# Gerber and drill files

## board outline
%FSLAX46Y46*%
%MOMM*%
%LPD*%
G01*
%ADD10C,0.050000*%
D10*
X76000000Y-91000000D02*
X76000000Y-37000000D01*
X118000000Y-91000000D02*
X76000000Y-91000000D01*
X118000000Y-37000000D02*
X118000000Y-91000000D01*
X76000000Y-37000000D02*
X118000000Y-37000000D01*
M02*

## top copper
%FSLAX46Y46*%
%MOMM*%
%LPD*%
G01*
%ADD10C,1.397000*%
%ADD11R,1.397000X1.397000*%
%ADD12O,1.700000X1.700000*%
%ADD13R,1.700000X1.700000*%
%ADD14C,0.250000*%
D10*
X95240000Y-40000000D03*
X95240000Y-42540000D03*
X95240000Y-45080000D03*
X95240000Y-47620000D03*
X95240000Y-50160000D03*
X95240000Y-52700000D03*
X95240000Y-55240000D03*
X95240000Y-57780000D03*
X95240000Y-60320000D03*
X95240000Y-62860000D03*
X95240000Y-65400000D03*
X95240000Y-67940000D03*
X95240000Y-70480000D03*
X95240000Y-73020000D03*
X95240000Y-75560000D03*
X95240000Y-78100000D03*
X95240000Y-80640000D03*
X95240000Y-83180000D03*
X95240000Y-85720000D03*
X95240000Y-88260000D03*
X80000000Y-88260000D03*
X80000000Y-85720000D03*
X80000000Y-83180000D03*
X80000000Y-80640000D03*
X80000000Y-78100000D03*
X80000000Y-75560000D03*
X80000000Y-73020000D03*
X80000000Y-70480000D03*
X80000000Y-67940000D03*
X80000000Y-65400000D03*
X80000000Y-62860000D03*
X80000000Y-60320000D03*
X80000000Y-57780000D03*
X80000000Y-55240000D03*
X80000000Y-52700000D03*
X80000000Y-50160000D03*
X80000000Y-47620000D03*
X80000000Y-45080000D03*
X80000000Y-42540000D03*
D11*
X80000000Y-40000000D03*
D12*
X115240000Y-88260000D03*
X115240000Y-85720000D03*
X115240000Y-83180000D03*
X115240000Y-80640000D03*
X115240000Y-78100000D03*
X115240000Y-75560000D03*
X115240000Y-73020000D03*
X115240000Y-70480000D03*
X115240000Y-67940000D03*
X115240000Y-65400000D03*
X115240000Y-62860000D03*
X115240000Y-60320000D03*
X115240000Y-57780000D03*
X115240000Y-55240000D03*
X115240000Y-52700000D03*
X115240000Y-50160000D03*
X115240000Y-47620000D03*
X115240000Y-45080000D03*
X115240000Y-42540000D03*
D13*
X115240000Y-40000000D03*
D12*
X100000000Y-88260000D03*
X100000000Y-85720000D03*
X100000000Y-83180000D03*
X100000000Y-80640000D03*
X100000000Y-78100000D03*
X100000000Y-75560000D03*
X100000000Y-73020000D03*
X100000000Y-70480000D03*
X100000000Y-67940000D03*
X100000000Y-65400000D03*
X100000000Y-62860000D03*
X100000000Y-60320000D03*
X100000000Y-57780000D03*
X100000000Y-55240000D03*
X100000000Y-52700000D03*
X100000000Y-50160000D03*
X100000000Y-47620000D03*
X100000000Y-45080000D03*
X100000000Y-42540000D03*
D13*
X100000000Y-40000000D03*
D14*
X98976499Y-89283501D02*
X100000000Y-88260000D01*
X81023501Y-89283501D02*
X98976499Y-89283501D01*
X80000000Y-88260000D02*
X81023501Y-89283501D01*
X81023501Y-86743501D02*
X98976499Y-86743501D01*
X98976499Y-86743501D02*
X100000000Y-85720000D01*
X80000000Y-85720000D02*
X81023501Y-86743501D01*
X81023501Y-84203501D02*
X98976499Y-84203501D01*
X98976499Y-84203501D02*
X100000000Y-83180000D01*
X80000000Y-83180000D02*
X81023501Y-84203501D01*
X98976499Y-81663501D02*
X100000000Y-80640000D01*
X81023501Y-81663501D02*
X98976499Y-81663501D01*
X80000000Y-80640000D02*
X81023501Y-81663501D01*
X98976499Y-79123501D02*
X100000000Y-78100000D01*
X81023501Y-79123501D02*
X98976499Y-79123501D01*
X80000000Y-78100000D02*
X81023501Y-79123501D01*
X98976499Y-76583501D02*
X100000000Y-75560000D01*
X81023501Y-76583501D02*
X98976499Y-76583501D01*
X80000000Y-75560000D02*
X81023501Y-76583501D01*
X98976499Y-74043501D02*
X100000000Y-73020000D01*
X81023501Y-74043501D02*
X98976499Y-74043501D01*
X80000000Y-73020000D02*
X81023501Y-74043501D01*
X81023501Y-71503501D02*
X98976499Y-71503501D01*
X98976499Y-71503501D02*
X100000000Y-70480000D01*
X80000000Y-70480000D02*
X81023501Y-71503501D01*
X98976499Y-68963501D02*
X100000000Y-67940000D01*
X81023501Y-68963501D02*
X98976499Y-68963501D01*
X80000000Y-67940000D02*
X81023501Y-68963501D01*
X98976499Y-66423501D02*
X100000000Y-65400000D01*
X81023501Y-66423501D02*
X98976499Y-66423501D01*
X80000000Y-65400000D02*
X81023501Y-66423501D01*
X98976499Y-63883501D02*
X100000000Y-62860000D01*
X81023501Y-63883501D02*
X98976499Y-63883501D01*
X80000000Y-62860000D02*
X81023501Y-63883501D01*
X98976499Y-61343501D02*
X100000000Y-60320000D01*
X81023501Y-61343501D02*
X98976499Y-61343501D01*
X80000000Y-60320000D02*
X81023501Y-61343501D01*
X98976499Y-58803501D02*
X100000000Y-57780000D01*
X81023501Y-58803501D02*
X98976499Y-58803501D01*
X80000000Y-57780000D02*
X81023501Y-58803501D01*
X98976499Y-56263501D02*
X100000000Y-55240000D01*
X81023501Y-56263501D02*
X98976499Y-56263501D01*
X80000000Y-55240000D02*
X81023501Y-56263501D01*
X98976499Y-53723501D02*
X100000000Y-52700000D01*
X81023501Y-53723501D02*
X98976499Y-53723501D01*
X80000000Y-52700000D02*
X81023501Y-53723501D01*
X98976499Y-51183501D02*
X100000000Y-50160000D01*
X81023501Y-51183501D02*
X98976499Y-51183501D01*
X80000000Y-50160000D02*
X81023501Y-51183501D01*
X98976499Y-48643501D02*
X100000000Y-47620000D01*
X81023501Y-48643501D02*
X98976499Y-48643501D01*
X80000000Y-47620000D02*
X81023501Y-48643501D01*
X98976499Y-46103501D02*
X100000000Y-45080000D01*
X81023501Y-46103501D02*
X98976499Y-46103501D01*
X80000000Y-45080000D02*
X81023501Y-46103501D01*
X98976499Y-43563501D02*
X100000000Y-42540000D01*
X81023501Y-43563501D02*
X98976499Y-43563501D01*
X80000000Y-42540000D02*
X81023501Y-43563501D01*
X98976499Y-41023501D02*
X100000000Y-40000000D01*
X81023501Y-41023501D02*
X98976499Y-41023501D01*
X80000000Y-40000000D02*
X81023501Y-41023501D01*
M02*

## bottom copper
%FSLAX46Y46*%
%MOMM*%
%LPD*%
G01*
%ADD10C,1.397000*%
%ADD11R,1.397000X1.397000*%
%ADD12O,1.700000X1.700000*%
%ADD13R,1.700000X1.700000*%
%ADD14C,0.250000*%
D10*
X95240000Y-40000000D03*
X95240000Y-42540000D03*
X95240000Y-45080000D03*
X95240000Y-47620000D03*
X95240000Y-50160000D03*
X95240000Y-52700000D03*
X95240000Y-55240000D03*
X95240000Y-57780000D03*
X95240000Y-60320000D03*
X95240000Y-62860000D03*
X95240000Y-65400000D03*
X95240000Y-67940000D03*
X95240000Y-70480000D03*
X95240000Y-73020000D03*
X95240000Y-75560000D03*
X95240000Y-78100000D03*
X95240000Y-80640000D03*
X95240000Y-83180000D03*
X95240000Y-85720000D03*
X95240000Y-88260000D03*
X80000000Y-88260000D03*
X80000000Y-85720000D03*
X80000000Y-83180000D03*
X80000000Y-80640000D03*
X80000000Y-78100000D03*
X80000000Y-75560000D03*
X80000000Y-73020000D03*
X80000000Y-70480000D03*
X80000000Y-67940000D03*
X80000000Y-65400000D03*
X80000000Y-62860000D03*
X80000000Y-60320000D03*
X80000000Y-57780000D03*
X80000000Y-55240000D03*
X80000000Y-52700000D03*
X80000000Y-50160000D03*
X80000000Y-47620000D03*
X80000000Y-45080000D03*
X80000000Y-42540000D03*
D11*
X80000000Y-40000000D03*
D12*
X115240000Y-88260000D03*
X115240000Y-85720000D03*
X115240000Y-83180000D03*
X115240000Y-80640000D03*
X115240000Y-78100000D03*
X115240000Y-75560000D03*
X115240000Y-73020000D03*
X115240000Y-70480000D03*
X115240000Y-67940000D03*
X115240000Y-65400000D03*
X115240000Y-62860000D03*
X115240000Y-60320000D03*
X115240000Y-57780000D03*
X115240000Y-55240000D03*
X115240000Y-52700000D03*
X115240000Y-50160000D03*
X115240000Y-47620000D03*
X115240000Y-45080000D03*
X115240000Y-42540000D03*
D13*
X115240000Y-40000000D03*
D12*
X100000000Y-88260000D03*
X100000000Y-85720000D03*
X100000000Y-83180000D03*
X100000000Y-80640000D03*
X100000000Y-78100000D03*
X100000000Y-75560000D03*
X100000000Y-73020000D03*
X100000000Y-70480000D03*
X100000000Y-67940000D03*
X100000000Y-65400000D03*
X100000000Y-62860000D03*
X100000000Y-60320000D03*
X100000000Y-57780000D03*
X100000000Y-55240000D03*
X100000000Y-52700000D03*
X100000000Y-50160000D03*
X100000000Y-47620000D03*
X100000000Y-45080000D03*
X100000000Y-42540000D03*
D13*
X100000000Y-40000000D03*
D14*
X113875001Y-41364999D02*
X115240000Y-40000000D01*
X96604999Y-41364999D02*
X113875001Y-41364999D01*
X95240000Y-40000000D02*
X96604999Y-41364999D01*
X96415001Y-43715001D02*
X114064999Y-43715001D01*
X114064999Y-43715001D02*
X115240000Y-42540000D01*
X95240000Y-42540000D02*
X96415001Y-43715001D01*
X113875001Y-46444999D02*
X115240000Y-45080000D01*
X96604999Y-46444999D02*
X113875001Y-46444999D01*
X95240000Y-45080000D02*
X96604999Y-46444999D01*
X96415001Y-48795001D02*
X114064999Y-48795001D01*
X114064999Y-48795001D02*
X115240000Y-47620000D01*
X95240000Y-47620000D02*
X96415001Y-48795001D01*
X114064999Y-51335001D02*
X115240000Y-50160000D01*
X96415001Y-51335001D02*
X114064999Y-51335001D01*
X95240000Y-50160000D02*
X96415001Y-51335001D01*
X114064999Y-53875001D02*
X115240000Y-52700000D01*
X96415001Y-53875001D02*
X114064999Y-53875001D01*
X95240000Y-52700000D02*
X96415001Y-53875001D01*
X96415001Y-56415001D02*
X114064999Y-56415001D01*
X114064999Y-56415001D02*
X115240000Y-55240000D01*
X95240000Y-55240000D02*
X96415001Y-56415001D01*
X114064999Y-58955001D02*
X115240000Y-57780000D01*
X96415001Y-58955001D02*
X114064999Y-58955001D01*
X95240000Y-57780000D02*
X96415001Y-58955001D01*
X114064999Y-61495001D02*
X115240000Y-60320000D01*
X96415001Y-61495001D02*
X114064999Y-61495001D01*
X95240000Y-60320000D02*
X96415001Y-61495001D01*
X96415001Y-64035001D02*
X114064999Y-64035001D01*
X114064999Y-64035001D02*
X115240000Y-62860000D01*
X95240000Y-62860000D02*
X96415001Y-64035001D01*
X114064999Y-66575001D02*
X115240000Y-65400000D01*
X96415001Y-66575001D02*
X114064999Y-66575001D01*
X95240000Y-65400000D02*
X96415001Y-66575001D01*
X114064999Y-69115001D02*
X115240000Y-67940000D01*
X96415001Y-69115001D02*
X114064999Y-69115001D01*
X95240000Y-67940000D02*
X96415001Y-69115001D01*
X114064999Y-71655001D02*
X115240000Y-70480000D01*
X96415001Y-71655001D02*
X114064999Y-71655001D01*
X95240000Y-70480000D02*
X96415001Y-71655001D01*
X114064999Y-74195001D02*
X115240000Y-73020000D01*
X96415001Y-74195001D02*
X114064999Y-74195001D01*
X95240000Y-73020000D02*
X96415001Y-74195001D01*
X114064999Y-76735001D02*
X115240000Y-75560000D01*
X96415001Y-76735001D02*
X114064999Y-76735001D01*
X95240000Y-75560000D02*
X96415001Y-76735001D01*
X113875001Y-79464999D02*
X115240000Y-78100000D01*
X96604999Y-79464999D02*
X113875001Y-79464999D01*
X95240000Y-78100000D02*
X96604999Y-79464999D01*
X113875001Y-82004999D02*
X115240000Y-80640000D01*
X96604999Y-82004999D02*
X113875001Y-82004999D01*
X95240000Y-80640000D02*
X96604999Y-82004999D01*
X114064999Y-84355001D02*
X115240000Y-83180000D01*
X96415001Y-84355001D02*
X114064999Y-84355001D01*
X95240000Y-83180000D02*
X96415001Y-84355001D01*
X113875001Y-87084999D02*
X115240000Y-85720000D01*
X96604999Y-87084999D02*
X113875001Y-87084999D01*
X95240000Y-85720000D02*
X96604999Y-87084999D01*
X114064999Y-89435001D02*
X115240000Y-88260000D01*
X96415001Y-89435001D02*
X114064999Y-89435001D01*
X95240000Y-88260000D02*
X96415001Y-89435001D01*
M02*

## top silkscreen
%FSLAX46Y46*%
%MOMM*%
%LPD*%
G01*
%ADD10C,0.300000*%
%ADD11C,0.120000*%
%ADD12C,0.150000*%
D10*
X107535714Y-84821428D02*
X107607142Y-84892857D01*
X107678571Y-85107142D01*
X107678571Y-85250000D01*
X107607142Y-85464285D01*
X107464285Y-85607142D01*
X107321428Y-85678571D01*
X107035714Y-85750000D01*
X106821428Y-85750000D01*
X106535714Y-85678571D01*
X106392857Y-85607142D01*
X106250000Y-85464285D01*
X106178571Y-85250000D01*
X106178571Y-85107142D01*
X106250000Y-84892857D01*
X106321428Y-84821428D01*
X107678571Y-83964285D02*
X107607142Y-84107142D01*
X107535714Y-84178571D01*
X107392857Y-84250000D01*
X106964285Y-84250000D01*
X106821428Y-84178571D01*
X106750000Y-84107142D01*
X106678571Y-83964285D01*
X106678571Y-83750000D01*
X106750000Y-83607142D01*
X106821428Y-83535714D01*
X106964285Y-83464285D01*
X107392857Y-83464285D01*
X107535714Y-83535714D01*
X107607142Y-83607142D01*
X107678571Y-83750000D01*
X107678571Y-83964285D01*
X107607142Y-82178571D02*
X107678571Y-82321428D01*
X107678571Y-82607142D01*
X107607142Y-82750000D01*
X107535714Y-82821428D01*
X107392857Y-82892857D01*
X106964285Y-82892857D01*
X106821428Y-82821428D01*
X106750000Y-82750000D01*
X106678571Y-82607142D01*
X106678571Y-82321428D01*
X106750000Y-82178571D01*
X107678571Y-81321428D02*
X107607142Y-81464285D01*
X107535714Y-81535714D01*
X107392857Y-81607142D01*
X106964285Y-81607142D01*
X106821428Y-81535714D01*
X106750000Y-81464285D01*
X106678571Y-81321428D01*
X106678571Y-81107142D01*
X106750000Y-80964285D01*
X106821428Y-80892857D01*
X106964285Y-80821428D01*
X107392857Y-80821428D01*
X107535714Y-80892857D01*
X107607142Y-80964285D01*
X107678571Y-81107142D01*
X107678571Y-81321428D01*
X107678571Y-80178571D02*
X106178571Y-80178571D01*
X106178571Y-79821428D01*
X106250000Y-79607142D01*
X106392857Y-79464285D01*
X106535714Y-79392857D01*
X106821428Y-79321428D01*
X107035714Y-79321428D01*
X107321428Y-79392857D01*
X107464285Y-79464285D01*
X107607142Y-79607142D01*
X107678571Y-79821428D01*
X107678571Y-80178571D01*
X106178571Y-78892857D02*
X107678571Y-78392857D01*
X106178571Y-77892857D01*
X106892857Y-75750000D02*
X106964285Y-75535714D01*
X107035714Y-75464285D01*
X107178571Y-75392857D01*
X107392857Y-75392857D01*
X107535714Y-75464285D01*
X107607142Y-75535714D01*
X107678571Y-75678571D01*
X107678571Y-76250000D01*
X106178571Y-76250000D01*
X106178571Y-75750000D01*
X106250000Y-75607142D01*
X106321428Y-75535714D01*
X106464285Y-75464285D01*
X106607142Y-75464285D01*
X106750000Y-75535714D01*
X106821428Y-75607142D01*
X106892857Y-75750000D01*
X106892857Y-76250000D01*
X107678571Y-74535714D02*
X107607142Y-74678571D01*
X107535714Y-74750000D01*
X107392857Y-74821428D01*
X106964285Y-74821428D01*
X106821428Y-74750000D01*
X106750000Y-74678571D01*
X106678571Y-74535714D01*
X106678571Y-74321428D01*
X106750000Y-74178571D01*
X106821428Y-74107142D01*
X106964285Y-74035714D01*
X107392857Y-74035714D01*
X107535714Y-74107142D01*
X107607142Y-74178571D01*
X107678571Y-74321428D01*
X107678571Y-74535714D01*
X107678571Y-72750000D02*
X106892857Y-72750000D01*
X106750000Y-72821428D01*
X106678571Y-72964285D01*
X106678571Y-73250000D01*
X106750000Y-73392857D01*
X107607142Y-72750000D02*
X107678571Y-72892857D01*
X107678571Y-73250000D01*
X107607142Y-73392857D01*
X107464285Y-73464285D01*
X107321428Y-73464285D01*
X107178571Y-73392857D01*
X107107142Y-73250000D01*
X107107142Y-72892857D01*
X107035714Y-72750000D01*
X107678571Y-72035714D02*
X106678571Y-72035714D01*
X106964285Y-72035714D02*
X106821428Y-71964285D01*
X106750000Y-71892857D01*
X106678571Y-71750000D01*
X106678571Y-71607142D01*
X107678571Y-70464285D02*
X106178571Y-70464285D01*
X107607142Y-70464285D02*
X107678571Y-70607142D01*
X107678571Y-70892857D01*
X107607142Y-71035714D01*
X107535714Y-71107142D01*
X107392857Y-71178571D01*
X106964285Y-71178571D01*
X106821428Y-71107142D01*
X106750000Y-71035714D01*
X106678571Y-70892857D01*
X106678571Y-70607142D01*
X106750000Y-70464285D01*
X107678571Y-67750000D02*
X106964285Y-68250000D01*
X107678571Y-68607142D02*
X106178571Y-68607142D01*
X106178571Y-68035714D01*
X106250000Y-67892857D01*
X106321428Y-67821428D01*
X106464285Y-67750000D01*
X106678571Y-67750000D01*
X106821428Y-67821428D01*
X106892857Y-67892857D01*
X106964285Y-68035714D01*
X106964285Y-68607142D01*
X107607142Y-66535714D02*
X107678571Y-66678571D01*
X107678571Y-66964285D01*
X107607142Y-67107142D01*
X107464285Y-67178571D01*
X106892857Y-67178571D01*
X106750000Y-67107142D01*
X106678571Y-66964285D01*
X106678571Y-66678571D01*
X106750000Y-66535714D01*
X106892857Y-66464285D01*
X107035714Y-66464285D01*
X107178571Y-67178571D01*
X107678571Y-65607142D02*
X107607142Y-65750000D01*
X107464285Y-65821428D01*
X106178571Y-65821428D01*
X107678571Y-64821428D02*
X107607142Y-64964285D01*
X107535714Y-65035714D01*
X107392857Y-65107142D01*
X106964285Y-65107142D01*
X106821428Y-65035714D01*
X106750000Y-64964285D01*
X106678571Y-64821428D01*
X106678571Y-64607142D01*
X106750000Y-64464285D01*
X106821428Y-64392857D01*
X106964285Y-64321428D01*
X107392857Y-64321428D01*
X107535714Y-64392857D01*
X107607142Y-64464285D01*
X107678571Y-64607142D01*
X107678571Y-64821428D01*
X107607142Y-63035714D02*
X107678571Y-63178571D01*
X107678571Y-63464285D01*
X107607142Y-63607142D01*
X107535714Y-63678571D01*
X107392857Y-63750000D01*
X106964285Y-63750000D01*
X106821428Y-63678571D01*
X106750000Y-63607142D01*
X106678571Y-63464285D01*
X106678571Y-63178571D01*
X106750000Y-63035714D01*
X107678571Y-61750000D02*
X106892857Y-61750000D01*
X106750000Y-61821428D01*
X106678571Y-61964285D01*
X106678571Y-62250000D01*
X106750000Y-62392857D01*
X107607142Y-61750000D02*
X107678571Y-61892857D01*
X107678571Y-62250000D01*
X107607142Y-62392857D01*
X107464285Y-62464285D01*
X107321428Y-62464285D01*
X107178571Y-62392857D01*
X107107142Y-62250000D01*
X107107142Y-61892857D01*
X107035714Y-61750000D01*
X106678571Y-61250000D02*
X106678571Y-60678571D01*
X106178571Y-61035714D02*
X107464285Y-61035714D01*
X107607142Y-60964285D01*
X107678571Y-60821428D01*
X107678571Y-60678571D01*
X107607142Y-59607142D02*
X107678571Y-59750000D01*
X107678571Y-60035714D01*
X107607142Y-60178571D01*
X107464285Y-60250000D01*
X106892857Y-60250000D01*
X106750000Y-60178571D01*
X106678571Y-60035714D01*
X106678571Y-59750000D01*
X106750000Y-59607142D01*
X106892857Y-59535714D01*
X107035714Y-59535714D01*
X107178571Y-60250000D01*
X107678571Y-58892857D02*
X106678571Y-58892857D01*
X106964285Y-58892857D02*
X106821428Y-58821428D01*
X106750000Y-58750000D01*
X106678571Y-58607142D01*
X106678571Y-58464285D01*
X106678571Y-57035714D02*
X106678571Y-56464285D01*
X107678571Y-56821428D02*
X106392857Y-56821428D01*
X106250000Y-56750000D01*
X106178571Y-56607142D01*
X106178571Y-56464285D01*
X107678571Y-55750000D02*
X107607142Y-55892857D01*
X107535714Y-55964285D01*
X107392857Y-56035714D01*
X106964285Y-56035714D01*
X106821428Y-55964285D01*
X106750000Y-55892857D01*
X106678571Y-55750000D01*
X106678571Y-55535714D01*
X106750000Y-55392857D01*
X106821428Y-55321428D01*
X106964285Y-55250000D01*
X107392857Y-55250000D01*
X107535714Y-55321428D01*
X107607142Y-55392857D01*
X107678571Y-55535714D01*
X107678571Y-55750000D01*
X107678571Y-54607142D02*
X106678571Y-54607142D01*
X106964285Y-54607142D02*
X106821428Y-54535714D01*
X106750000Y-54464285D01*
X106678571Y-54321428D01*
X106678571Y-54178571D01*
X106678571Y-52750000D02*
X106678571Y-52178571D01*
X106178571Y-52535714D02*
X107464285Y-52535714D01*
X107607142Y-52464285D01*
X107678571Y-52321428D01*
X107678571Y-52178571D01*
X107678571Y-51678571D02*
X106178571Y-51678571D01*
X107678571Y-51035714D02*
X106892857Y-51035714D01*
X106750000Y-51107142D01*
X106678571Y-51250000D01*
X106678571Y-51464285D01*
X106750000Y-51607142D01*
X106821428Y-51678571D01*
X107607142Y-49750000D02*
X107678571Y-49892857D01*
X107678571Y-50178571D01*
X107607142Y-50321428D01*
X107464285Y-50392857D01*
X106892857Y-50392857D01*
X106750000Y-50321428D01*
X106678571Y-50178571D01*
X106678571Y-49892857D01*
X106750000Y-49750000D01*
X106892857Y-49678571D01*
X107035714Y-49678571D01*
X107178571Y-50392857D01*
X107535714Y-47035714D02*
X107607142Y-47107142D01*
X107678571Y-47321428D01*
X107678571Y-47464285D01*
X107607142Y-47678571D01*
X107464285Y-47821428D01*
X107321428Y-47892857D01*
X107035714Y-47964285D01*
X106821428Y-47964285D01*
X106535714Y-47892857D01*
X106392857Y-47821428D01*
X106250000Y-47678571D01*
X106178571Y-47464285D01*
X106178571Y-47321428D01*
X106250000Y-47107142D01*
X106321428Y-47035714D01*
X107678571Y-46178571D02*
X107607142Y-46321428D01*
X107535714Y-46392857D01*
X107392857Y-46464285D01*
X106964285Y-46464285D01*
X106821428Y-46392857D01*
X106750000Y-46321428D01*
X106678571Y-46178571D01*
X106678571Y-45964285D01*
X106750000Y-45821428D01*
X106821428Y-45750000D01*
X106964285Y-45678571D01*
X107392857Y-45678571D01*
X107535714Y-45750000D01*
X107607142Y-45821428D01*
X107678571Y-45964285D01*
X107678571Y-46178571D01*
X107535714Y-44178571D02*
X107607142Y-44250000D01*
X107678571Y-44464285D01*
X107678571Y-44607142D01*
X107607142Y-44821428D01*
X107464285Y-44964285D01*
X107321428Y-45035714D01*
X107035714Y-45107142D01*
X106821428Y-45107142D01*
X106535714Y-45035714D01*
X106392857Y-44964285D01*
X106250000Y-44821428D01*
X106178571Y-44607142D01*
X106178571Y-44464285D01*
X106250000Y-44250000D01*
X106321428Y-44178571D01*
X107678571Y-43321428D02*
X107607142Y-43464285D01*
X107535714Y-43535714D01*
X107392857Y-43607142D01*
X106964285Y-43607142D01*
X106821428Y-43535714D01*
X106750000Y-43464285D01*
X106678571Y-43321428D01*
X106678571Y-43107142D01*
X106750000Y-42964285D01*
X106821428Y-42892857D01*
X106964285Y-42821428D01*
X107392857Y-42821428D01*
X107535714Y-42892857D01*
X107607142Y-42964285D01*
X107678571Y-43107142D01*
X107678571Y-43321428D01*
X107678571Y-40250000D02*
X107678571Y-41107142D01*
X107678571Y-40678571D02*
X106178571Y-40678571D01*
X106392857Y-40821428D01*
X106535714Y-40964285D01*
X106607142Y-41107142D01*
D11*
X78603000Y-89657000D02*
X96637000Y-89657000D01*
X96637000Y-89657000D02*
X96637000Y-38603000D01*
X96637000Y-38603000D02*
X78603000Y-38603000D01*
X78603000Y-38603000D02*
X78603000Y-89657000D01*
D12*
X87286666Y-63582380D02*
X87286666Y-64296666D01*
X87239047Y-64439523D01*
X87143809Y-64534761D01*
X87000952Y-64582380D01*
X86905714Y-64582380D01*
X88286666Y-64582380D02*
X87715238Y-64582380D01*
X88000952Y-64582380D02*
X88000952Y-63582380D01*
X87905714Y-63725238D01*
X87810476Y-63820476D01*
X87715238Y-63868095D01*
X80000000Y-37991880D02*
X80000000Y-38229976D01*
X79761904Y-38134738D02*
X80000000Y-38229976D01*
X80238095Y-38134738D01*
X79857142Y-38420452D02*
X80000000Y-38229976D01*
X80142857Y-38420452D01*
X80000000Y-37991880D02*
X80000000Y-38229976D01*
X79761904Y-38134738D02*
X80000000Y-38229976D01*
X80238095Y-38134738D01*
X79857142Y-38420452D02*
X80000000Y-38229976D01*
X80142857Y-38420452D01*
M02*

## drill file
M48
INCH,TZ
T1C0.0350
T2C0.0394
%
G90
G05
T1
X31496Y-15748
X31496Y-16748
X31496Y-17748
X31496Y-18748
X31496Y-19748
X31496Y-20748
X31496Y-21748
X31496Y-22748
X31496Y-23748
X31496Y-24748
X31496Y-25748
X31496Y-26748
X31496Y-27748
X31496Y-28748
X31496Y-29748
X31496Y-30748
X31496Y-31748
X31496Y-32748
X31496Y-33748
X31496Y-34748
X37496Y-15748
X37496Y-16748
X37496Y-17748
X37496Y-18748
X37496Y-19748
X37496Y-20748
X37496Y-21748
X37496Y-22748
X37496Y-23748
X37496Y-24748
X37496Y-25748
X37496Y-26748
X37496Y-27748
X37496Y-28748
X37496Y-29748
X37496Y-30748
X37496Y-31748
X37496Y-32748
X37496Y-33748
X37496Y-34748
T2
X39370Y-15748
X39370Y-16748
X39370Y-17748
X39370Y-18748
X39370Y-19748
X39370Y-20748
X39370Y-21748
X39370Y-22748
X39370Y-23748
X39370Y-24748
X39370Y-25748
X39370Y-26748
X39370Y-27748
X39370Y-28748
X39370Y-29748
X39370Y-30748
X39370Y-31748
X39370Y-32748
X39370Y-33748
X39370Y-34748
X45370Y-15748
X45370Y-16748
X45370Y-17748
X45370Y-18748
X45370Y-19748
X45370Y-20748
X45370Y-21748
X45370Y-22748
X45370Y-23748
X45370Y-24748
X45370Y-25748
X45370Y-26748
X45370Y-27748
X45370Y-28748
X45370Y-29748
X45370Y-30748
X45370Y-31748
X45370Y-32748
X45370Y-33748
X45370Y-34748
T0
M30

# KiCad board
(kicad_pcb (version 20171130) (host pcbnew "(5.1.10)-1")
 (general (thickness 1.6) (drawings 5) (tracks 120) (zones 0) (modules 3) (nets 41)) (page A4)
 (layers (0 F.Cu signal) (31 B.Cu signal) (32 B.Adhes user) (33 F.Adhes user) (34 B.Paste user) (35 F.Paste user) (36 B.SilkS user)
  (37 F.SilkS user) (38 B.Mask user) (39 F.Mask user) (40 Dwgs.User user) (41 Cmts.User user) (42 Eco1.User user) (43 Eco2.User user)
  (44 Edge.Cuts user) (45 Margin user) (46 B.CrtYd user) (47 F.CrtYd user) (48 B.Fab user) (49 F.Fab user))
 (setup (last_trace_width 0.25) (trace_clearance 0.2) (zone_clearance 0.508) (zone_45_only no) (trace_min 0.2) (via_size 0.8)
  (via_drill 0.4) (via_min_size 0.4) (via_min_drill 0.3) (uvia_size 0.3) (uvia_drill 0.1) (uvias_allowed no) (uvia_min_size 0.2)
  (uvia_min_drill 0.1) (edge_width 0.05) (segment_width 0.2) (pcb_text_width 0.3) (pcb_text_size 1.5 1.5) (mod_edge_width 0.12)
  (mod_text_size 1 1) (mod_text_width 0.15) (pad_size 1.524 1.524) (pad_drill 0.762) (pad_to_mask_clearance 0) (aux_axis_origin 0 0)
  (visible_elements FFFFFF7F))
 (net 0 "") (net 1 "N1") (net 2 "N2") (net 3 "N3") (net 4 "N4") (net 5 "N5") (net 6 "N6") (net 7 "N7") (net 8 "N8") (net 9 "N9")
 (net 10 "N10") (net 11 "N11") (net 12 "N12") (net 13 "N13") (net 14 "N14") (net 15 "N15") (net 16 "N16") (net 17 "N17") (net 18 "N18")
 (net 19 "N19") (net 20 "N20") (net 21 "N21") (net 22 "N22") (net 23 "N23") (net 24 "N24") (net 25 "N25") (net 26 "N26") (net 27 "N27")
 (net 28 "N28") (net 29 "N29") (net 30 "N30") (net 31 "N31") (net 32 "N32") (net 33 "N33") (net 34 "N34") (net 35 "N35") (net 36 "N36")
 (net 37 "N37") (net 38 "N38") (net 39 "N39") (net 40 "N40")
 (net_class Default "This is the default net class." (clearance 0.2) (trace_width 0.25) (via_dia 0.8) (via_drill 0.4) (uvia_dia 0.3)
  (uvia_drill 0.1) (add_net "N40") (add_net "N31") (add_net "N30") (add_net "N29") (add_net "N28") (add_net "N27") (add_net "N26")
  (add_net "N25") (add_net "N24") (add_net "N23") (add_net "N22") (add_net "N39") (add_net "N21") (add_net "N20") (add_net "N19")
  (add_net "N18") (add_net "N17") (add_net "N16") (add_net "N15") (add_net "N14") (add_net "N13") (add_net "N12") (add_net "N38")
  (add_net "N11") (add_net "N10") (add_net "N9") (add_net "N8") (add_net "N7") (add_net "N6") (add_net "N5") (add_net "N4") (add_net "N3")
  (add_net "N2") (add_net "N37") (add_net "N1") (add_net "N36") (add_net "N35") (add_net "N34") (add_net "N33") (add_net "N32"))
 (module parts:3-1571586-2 (layer F.Cu) (at 80 40)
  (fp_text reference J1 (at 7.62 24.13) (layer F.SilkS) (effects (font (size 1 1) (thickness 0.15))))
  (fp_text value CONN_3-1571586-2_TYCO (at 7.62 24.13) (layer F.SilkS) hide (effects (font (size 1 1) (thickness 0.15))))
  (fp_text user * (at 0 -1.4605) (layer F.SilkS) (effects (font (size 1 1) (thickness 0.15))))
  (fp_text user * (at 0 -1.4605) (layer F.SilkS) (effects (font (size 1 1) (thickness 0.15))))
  (fp_line (start -1.397 49.657) (end 16.637 49.657) (layer F.SilkS) (width 0.12))
  (fp_line (start 16.637 49.657) (end 16.637 -1.397) (layer F.SilkS) (width 0.12))
  (fp_line (start 16.637 -1.397) (end -1.397 -1.397) (layer F.SilkS) (width 0.12))
  (fp_line (start -1.397 -1.397) (end -1.397 49.657) (layer F.SilkS) (width 0.12))
  (pad 40 thru_hole circle (at 15.24 0) (size 1.397 1.397) (drill 0.889) (layers *.Cu *.Mask) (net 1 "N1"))
  (pad 39 thru_hole circle (at 15.24 2.54) (size 1.397 1.397) (drill 0.889) (layers *.Cu *.Mask) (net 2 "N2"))
  (pad 38 thru_hole circle (at 15.24 5.08) (size 1.397 1.397) (drill 0.889) (layers *.Cu *.Mask) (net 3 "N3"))
  (pad 37 thru_hole circle (at 15.24 7.62) (size 1.397 1.397) (drill 0.889) (layers *.Cu *.Mask) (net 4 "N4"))
  (pad 36 thru_hole circle (at 15.24 10.16) (size 1.397 1.397) (drill 0.889) (layers *.Cu *.Mask) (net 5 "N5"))
  (pad 35 thru_hole circle (at 15.24 12.7) (size 1.397 1.397) (drill 0.889) (layers *.Cu *.Mask) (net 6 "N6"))
  (pad 34 thru_hole circle (at 15.24 15.24) (size 1.397 1.397) (drill 0.889) (layers *.Cu *.Mask) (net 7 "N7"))
  (pad 33 thru_hole circle (at 15.24 17.78) (size 1.397 1.397) (drill 0.889) (layers *.Cu *.Mask) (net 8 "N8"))
  (pad 32 thru_hole circle (at 15.24 20.32) (size 1.397 1.397) (drill 0.889) (layers *.Cu *.Mask) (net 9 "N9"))
  (pad 31 thru_hole circle (at 15.24 22.86) (size 1.397 1.397) (drill 0.889) (layers *.Cu *.Mask) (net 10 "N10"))
  (pad 30 thru_hole circle (at 15.24 25.4) (size 1.397 1.397) (drill 0.889) (layers *.Cu *.Mask) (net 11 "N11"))
  (pad 29 thru_hole circle (at 15.24 27.94) (size 1.397 1.397) (drill 0.889) (layers *.Cu *.Mask) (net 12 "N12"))
  (pad 28 thru_hole circle (at 15.24 30.48) (size 1.397 1.397) (drill 0.889) (layers *.Cu *.Mask) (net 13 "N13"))
  (pad 27 thru_hole circle (at 15.24 33.02) (size 1.397 1.397) (drill 0.889) (layers *.Cu *.Mask) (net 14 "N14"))
  (pad 26 thru_hole circle (at 15.24 35.56) (size 1.397 1.397) (drill 0.889) (layers *.Cu *.Mask) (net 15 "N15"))
  (pad 25 thru_hole circle (at 15.24 38.1) (size 1.397 1.397) (drill 0.889) (layers *.Cu *.Mask) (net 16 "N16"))
  (pad 24 thru_hole circle (at 15.24 40.64) (size 1.397 1.397) (drill 0.889) (layers *.Cu *.Mask) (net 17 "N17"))
  (pad 23 thru_hole circle (at 15.24 43.18) (size 1.397 1.397) (drill 0.889) (layers *.Cu *.Mask) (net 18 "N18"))
  (pad 22 thru_hole circle (at 15.24 45.72) (size 1.397 1.397) (drill 0.889) (layers *.Cu *.Mask) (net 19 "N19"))
  (pad 21 thru_hole circle (at 15.24 48.26) (size 1.397 1.397) (drill 0.889) (layers *.Cu *.Mask) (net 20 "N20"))
  (pad 20 thru_hole circle (at 0 48.26) (size 1.397 1.397) (drill 0.889) (layers *.Cu *.Mask) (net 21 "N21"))
  (pad 19 thru_hole circle (at 0 45.72) (size 1.397 1.397) (drill 0.889) (layers *.Cu *.Mask) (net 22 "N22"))
  (pad 18 thru_hole circle (at 0 43.18) (size 1.397 1.397) (drill 0.889) (layers *.Cu *.Mask) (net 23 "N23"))
  (pad 17 thru_hole circle (at 0 40.64) (size 1.397 1.397) (drill 0.889) (layers *.Cu *.Mask) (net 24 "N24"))
  (pad 16 thru_hole circle (at 0 38.1) (size 1.397 1.397) (drill 0.889) (layers *.Cu *.Mask) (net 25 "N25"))
  (pad 15 thru_hole circle (at 0 35.56) (size 1.397 1.397) (drill 0.889) (layers *.Cu *.Mask) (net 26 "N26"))
  (pad 14 thru_hole circle (at 0 33.02) (size 1.397 1.397) (drill 0.889) (layers *.Cu *.Mask) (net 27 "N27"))
  (pad 13 thru_hole circle (at 0 30.48) (size 1.397 1.397) (drill 0.889) (layers *.Cu *.Mask) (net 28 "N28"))
  (pad 12 thru_hole circle (at 0 27.94) (size 1.397 1.397) (drill 0.889) (layers *.Cu *.Mask) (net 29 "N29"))
  (pad 11 thru_hole circle (at 0 25.4) (size 1.397 1.397) (drill 0.889) (layers *.Cu *.Mask) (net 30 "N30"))
  (pad 10 thru_hole circle (at 0 22.86) (size 1.397 1.397) (drill 0.889) (layers *.Cu *.Mask) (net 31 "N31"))
  (pad 9 thru_hole circle (at 0 20.32) (size 1.397 1.397) (drill 0.889) (layers *.Cu *.Mask) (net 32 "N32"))
  (pad 8 thru_hole circle (at 0 17.78) (size 1.397 1.397) (drill 0.889) (layers *.Cu *.Mask) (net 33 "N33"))
  (pad 7 thru_hole circle (at 0 15.24) (size 1.397 1.397) (drill 0.889) (layers *.Cu *.Mask) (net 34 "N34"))
  (pad 6 thru_hole circle (at 0 12.7) (size 1.397 1.397) (drill 0.889) (layers *.Cu *.Mask) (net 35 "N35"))
  (pad 5 thru_hole circle (at 0 10.16) (size 1.397 1.397) (drill 0.889) (layers *.Cu *.Mask) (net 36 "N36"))
  (pad 4 thru_hole circle (at 0 7.62) (size 1.397 1.397) (drill 0.889) (layers *.Cu *.Mask) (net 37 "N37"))
  (pad 3 thru_hole circle (at 0 5.08) (size 1.397 1.397) (drill 0.889) (layers *.Cu *.Mask) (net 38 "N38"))
  (pad 2 thru_hole circle (at 0 2.54) (size 1.397 1.397) (drill 0.889) (layers *.Cu *.Mask) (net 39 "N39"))
  (pad 1 thru_hole rect (at 0 0) (size 1.397 1.397) (drill 0.889) (layers *.Cu *.Mask) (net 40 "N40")))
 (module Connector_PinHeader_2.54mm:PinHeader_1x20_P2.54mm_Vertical (layer B.Cu) (at 115.24 40 180)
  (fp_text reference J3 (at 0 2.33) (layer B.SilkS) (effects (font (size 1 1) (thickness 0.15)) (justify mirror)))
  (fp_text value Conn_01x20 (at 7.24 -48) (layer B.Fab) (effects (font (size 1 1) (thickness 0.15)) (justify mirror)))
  (pad 20 thru_hole oval (at 0 -48.26 180) (size 1.7 1.7) (drill 1) (layers *.Cu *.Mask) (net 20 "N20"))
  (pad 19 thru_hole oval (at 0 -45.72 180) (size 1.7 1.7) (drill 1) (layers *.Cu *.Mask) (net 19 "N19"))
  (pad 18 thru_hole oval (at 0 -43.18 180) (size 1.7 1.7) (drill 1) (layers *.Cu *.Mask) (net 18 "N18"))
  (pad 17 thru_hole oval (at 0 -40.64 180) (size 1.7 1.7) (drill 1) (layers *.Cu *.Mask) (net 17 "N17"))
  (pad 16 thru_hole oval (at 0 -38.1 180) (size 1.7 1.7) (drill 1) (layers *.Cu *.Mask) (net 16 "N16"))
  (pad 15 thru_hole oval (at 0 -35.56 180) (size 1.7 1.7) (drill 1) (layers *.Cu *.Mask) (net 15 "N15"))
  (pad 14 thru_hole oval (at 0 -33.02 180) (size 1.7 1.7) (drill 1) (layers *.Cu *.Mask) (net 14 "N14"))
  (pad 13 thru_hole oval (at 0 -30.48 180) (size 1.7 1.7) (drill 1) (layers *.Cu *.Mask) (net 13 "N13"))
  (pad 12 thru_hole oval (at 0 -27.94 180) (size 1.7 1.7) (drill 1) (layers *.Cu *.Mask) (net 12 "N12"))
  (pad 11 thru_hole oval (at 0 -25.4 180) (size 1.7 1.7) (drill 1) (layers *.Cu *.Mask) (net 11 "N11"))
  (pad 10 thru_hole oval (at 0 -22.86 180) (size 1.7 1.7) (drill 1) (layers *.Cu *.Mask) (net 10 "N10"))
  (pad 9 thru_hole oval (at 0 -20.32 180) (size 1.7 1.7) (drill 1) (layers *.Cu *.Mask) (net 9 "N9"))
  (pad 8 thru_hole oval (at 0 -17.78 180) (size 1.7 1.7) (drill 1) (layers *.Cu *.Mask) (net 8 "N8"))
  (pad 7 thru_hole oval (at 0 -15.24 180) (size 1.7 1.7) (drill 1) (layers *.Cu *.Mask) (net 7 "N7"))
  (pad 6 thru_hole oval (at 0 -12.7 180) (size 1.7 1.7) (drill 1) (layers *.Cu *.Mask) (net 6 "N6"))
  (pad 5 thru_hole oval (at 0 -10.16 180) (size 1.7 1.7) (drill 1) (layers *.Cu *.Mask) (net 5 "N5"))
  (pad 4 thru_hole oval (at 0 -7.62 180) (size 1.7 1.7) (drill 1) (layers *.Cu *.Mask) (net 4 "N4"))
  (pad 3 thru_hole oval (at 0 -5.08 180) (size 1.7 1.7) (drill 1) (layers *.Cu *.Mask) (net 3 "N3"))
  (pad 2 thru_hole oval (at 0 -2.54 180) (size 1.7 1.7) (drill 1) (layers *.Cu *.Mask) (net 2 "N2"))
  (pad 1 thru_hole rect (at 0 0 180) (size 1.7 1.7) (drill 1) (layers *.Cu *.Mask) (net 1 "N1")))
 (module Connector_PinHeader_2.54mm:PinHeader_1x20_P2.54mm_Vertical (layer B.Cu) (at 100 40 180)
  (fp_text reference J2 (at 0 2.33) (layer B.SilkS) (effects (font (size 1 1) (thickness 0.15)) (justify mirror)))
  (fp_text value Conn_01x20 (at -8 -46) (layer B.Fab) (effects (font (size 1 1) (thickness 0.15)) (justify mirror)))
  (pad 20 thru_hole oval (at 0 -48.26 180) (size 1.7 1.7) (drill 1) (layers *.Cu *.Mask) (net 21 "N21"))
  (pad 19 thru_hole oval (at 0 -45.72 180) (size 1.7 1.7) (drill 1) (layers *.Cu *.Mask) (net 22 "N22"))
  (pad 18 thru_hole oval (at 0 -43.18 180) (size 1.7 1.7) (drill 1) (layers *.Cu *.Mask) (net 23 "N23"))
  (pad 17 thru_hole oval (at 0 -40.64 180) (size 1.7 1.7) (drill 1) (layers *.Cu *.Mask) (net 24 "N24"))
  (pad 16 thru_hole oval (at 0 -38.1 180) (size 1.7 1.7) (drill 1) (layers *.Cu *.Mask) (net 25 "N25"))
  (pad 15 thru_hole oval (at 0 -35.56 180) (size 1.7 1.7) (drill 1) (layers *.Cu *.Mask) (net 26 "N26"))
  (pad 14 thru_hole oval (at 0 -33.02 180) (size 1.7 1.7) (drill 1) (layers *.Cu *.Mask) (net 27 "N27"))
  (pad 13 thru_hole oval (at 0 -30.48 180) (size 1.7 1.7) (drill 1) (layers *.Cu *.Mask) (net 28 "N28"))
  (pad 12 thru_hole oval (at 0 -27.94 180) (size 1.7 1.7) (drill 1) (layers *.Cu *.Mask) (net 29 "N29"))
  (pad 11 thru_hole oval (at 0 -25.4 180) (size 1.7 1.7) (drill 1) (layers *.Cu *.Mask) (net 30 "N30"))
  (pad 10 thru_hole oval (at 0 -22.86 180) (size 1.7 1.7) (drill 1) (layers *.Cu *.Mask) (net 31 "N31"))
  (pad 9 thru_hole oval (at 0 -20.32 180) (size 1.7 1.7) (drill 1) (layers *.Cu *.Mask) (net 32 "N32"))
  (pad 8 thru_hole oval (at 0 -17.78 180) (size 1.7 1.7) (drill 1) (layers *.Cu *.Mask) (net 33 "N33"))
  (pad 7 thru_hole oval (at 0 -15.24 180) (size 1.7 1.7) (drill 1) (layers *.Cu *.Mask) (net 34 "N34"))
  (pad 6 thru_hole oval (at 0 -12.7 180) (size 1.7 1.7) (drill 1) (layers *.Cu *.Mask) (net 35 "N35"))
  (pad 5 thru_hole oval (at 0 -10.16 180) (size 1.7 1.7) (drill 1) (layers *.Cu *.Mask) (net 36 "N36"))
  (pad 4 thru_hole oval (at 0 -7.62 180) (size 1.7 1.7) (drill 1) (layers *.Cu *.Mask) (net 37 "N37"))
  (pad 3 thru_hole oval (at 0 -5.08 180) (size 1.7 1.7) (drill 1) (layers *.Cu *.Mask) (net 38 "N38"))
  (pad 2 thru_hole oval (at 0 -2.54 180) (size 1.7 1.7) (drill 1) (layers *.Cu *.Mask) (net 39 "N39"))
  (pad 1 thru_hole rect (at 0 0 180) (size 1.7 1.7) (drill 1) (layers *.Cu *.Mask) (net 40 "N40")))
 (gr_line (start 76 91) (end 76 37) (layer Edge.Cuts) (width 0.05))
 (gr_line (start 118 91) (end 76 91) (layer Edge.Cuts) (width 0.05))
 (gr_line (start 118 37) (end 118 91) (layer Edge.Cuts) (width 0.05))
 (gr_line (start 76 37) (end 118 37) (layer Edge.Cuts) (width 0.05))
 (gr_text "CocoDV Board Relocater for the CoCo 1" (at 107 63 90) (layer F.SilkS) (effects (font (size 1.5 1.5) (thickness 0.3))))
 (segment (start 113.875001 41.364999) (end 115.24 40) (width 0.25) (layer B.Cu) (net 1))
 (segment (start 96.604999 41.364999) (end 113.875001 41.364999) (width 0.25) (layer B.Cu) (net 1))
 (segment (start 95.24 40) (end 96.604999 41.364999) (width 0.25) (layer B.Cu) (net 1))
 (segment (start 96.415001 43.715001) (end 114.064999 43.715001) (width 0.25) (layer B.Cu) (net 2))
 (segment (start 114.064999 43.715001) (end 115.24 42.54) (width 0.25) (layer B.Cu) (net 2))
 (segment (start 95.24 42.54) (end 96.415001 43.715001) (width 0.25) (layer B.Cu) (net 2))
 (segment (start 113.875001 46.444999) (end 115.24 45.08) (width 0.25) (layer B.Cu) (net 3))
 (segment (start 96.604999 46.444999) (end 113.875001 46.444999) (width 0.25) (layer B.Cu) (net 3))
 (segment (start 95.24 45.08) (end 96.604999 46.444999) (width 0.25) (layer B.Cu) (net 3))
 (segment (start 96.415001 48.795001) (end 114.064999 48.795001) (width 0.25) (layer B.Cu) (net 4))
 (segment (start 114.064999 48.795001) (end 115.24 47.62) (width 0.25) (layer B.Cu) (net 4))
 (segment (start 95.24 47.62) (end 96.415001 48.795001) (width 0.25) (layer B.Cu) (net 4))
 (segment (start 114.064999 51.335001) (end 115.24 50.16) (width 0.25) (layer B.Cu) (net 5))
 (segment (start 96.415001 51.335001) (end 114.064999 51.335001) (width 0.25) (layer B.Cu) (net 5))
 (segment (start 95.24 50.16) (end 96.415001 51.335001) (width 0.25) (layer B.Cu) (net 5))
 (segment (start 114.064999 53.875001) (end 115.24 52.7) (width 0.25) (layer B.Cu) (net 6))
 (segment (start 96.415001 53.875001) (end 114.064999 53.875001) (width 0.25) (layer B.Cu) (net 6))
 (segment (start 95.24 52.7) (end 96.415001 53.875001) (width 0.25) (layer B.Cu) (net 6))
 (segment (start 96.415001 56.415001) (end 114.064999 56.415001) (width 0.25) (layer B.Cu) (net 7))
 (segment (start 114.064999 56.415001) (end 115.24 55.24) (width 0.25) (layer B.Cu) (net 7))
 (segment (start 95.24 55.24) (end 96.415001 56.415001) (width 0.25) (layer B.Cu) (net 7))
 (segment (start 114.064999 58.955001) (end 115.24 57.78) (width 0.25) (layer B.Cu) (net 8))
 (segment (start 96.415001 58.955001) (end 114.064999 58.955001) (width 0.25) (layer B.Cu) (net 8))
 (segment (start 95.24 57.78) (end 96.415001 58.955001) (width 0.25) (layer B.Cu) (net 8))
 (segment (start 114.064999 61.495001) (end 115.24 60.32) (width 0.25) (layer B.Cu) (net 9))
 (segment (start 96.415001 61.495001) (end 114.064999 61.495001) (width 0.25) (layer B.Cu) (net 9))
 (segment (start 95.24 60.32) (end 96.415001 61.495001) (width 0.25) (layer B.Cu) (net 9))
 (segment (start 96.415001 64.035001) (end 114.064999 64.035001) (width 0.25) (layer B.Cu) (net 10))
 (segment (start 114.064999 64.035001) (end 115.24 62.86) (width 0.25) (layer B.Cu) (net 10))
 (segment (start 95.24 62.86) (end 96.415001 64.035001) (width 0.25) (layer B.Cu) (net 10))
 (segment (start 114.064999 66.575001) (end 115.24 65.4) (width 0.25) (layer B.Cu) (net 11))
 (segment (start 96.415001 66.575001) (end 114.064999 66.575001) (width 0.25) (layer B.Cu) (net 11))
 (segment (start 95.24 65.4) (end 96.415001 66.575001) (width 0.25) (layer B.Cu) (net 11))
 (segment (start 114.064999 69.115001) (end 115.24 67.94) (width 0.25) (layer B.Cu) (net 12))
 (segment (start 96.415001 69.115001) (end 114.064999 69.115001) (width 0.25) (layer B.Cu) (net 12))
 (segment (start 95.24 67.94) (end 96.415001 69.115001) (width 0.25) (layer B.Cu) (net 12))
 (segment (start 114.064999 71.655001) (end 115.24 70.48) (width 0.25) (layer B.Cu) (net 13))
 (segment (start 96.415001 71.655001) (end 114.064999 71.655001) (width 0.25) (layer B.Cu) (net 13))
 (segment (start 95.24 70.48) (end 96.415001 71.655001) (width 0.25) (layer B.Cu) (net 13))
 (segment (start 114.064999 74.195001) (end 115.24 73.02) (width 0.25) (layer B.Cu) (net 14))
 (segment (start 96.415001 74.195001) (end 114.064999 74.195001) (width 0.25) (layer B.Cu) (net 14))
 (segment (start 95.24 73.02) (end 96.415001 74.195001) (width 0.25) (layer B.Cu) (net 14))
 (segment (start 114.064999 76.735001) (end 115.24 75.56) (width 0.25) (layer B.Cu) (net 15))
 (segment (start 96.415001 76.735001) (end 114.064999 76.735001) (width 0.25) (layer B.Cu) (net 15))
 (segment (start 95.24 75.56) (end 96.415001 76.735001) (width 0.25) (layer B.Cu) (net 15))
 (segment (start 113.875001 79.464999) (end 115.24 78.1) (width 0.25) (layer B.Cu) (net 16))
 (segment (start 96.604999 79.464999) (end 113.875001 79.464999) (width 0.25) (layer B.Cu) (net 16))
 (segment (start 95.24 78.1) (end 96.604999 79.464999) (width 0.25) (layer B.Cu) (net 16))
 (segment (start 113.875001 82.004999) (end 115.24 80.64) (width 0.25) (layer B.Cu) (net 17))
 (segment (start 96.604999 82.004999) (end 113.875001 82.004999) (width 0.25) (layer B.Cu) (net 17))
 (segment (start 95.24 80.64) (end 96.604999 82.004999) (width 0.25) (layer B.Cu) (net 17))
 (segment (start 114.064999 84.355001) (end 115.24 83.18) (width 0.25) (layer B.Cu) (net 18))
 (segment (start 96.415001 84.355001) (end 114.064999 84.355001) (width 0.25) (layer B.Cu) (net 18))
 (segment (start 95.24 83.18) (end 96.415001 84.355001) (width 0.25) (layer B.Cu) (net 18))
 (segment (start 113.875001 87.084999) (end 115.24 85.72) (width 0.25) (layer B.Cu) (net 19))
 (segment (start 96.604999 87.084999) (end 113.875001 87.084999) (width 0.25) (layer B.Cu) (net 19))
 (segment (start 95.24 85.72) (end 96.604999 87.084999) (width 0.25) (layer B.Cu) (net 19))
 (segment (start 114.064999 89.435001) (end 115.24 88.26) (width 0.25) (layer B.Cu) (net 20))
 (segment (start 96.415001 89.435001) (end 114.064999 89.435001) (width 0.25) (layer B.Cu) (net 20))
 (segment (start 95.24 88.26) (end 96.415001 89.435001) (width 0.25) (layer B.Cu) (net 20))
 (segment (start 98.976499 89.283501) (end 100 88.26) (width 0.25) (layer F.Cu) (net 21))
 (segment (start 81.023501 89.283501) (end 98.976499 89.283501) (width 0.25) (layer F.Cu) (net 21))
 (segment (start 80 88.26) (end 81.023501 89.283501) (width 0.25) (layer F.Cu) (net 21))
 (segment (start 81.023501 86.743501) (end 98.976499 86.743501) (width 0.25) (layer F.Cu) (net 22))
 (segment (start 98.976499 86.743501) (end 100 85.72) (width 0.25) (layer F.Cu) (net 22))
 (segment (start 80 85.72) (end 81.023501 86.743501) (width 0.25) (layer F.Cu) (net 22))
 (segment (start 81.023501 84.203501) (end 98.976499 84.203501) (width 0.25) (layer F.Cu) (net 23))
 (segment (start 98.976499 84.203501) (end 100 83.18) (width 0.25) (layer F.Cu) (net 23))
 (segment (start 80 83.18) (end 81.023501 84.203501) (width 0.25) (layer F.Cu) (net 23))
 (segment (start 98.976499 81.663501) (end 100 80.64) (width 0.25) (layer F.Cu) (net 24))
 (segment (start 81.023501 81.663501) (end 98.976499 81.663501) (width 0.25) (layer F.Cu) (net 24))
 (segment (start 80 80.64) (end 81.023501 81.663501) (width 0.25) (layer F.Cu) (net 24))
 (segment (start 98.976499 79.123501) (end 100 78.1) (width 0.25) (layer F.Cu) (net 25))
 (segment (start 81.023501 79.123501) (end 98.976499 79.123501) (width 0.25) (layer F.Cu) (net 25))
 (segment (start 80 78.1) (end 81.023501 79.123501) (width 0.25) (layer F.Cu) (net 25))
 (segment (start 98.976499 76.583501) (end 100 75.56) (width 0.25) (layer F.Cu) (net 26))
 (segment (start 81.023501 76.583501) (end 98.976499 76.583501) (width 0.25) (layer F.Cu) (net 26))
 (segment (start 80 75.56) (end 81.023501 76.583501) (width 0.25) (layer F.Cu) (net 26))
 (segment (start 98.976499 74.043501) (end 100 73.02) (width 0.25) (layer F.Cu) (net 27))
 (segment (start 81.023501 74.043501) (end 98.976499 74.043501) (width 0.25) (layer F.Cu) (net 27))
 (segment (start 80 73.02) (end 81.023501 74.043501) (width 0.25) (layer F.Cu) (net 27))
 (segment (start 81.023501 71.503501) (end 98.976499 71.503501) (width 0.25) (layer F.Cu) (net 28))
 (segment (start 98.976499 71.503501) (end 100 70.48) (width 0.25) (layer F.Cu) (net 28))
 (segment (start 80 70.48) (end 81.023501 71.503501) (width 0.25) (layer F.Cu) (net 28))
 (segment (start 98.976499 68.963501) (end 100 67.94) (width 0.25) (layer F.Cu) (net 29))
 (segment (start 81.023501 68.963501) (end 98.976499 68.963501) (width 0.25) (layer F.Cu) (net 29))
 (segment (start 80 67.94) (end 81.023501 68.963501) (width 0.25) (layer F.Cu) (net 29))
 (segment (start 98.976499 66.423501) (end 100 65.4) (width 0.25) (layer F.Cu) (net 30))
 (segment (start 81.023501 66.423501) (end 98.976499 66.423501) (width 0.25) (layer F.Cu) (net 30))
 (segment (start 80 65.4) (end 81.023501 66.423501) (width 0.25) (layer F.Cu) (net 30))
 (segment (start 98.976499 63.883501) (end 100 62.86) (width 0.25) (layer F.Cu) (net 31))
 (segment (start 81.023501 63.883501) (end 98.976499 63.883501) (width 0.25) (layer F.Cu) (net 31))
 (segment (start 80 62.86) (end 81.023501 63.883501) (width 0.25) (layer F.Cu) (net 31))
 (segment (start 98.976499 61.343501) (end 100 60.32) (width 0.25) (layer F.Cu) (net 32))
 (segment (start 81.023501 61.343501) (end 98.976499 61.343501) (width 0.25) (layer F.Cu) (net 32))
 (segment (start 80 60.32) (end 81.023501 61.343501) (width 0.25) (layer F.Cu) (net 32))
 (segment (start 98.976499 58.803501) (end 100 57.78) (width 0.25) (layer F.Cu) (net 33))
 (segment (start 81.023501 58.803501) (end 98.976499 58.803501) (width 0.25) (layer F.Cu) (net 33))
 (segment (start 80 57.78) (end 81.023501 58.803501) (width 0.25) (layer F.Cu) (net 33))
 (segment (start 98.976499 56.263501) (end 100 55.24) (width 0.25) (layer F.Cu) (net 34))
 (segment (start 81.023501 56.263501) (end 98.976499 56.263501) (width 0.25) (layer F.Cu) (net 34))
 (segment (start 80 55.24) (end 81.023501 56.263501) (width 0.25) (layer F.Cu) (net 34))
 (segment (start 98.976499 53.723501) (end 100 52.7) (width 0.25) (layer F.Cu) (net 35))
 (segment (start 81.023501 53.723501) (end 98.976499 53.723501) (width 0.25) (layer F.Cu) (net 35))
 (segment (start 80 52.7) (end 81.023501 53.723501) (width 0.25) (layer F.Cu) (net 35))
 (segment (start 98.976499 51.183501) (end 100 50.16) (width 0.25) (layer F.Cu) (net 36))
 (segment (start 81.023501 51.183501) (end 98.976499 51.183501) (width 0.25) (layer F.Cu) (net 36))
 (segment (start 80 50.16) (end 81.023501 51.183501) (width 0.25) (layer F.Cu) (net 36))
 (segment (start 98.976499 48.643501) (end 100 47.62) (width 0.25) (layer F.Cu) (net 37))
 (segment (start 81.023501 48.643501) (end 98.976499 48.643501) (width 0.25) (layer F.Cu) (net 37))
 (segment (start 80 47.62) (end 81.023501 48.643501) (width 0.25) (layer F.Cu) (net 37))
 (segment (start 98.976499 46.103501) (end 100 45.08) (width 0.25) (layer F.Cu) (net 38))
 (segment (start 81.023501 46.103501) (end 98.976499 46.103501) (width 0.25) (layer F.Cu) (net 38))
 (segment (start 80 45.08) (end 81.023501 46.103501) (width 0.25) (layer F.Cu) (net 38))
 (segment (start 98.976499 43.563501) (end 100 42.54) (width 0.25) (layer F.Cu) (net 39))
 (segment (start 81.023501 43.563501) (end 98.976499 43.563501) (width 0.25) (layer F.Cu) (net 39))
 (segment (start 80 42.54) (end 81.023501 43.563501) (width 0.25) (layer F.Cu) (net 39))
 (segment (start 98.976499 41.023501) (end 100 40) (width 0.25) (layer F.Cu) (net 40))
 (segment (start 81.023501 41.023501) (end 98.976499 41.023501) (width 0.25) (layer F.Cu) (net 40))
 (segment (start 80 40) (end 81.023501 41.023501) (width 0.25) (layer F.Cu) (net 40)))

